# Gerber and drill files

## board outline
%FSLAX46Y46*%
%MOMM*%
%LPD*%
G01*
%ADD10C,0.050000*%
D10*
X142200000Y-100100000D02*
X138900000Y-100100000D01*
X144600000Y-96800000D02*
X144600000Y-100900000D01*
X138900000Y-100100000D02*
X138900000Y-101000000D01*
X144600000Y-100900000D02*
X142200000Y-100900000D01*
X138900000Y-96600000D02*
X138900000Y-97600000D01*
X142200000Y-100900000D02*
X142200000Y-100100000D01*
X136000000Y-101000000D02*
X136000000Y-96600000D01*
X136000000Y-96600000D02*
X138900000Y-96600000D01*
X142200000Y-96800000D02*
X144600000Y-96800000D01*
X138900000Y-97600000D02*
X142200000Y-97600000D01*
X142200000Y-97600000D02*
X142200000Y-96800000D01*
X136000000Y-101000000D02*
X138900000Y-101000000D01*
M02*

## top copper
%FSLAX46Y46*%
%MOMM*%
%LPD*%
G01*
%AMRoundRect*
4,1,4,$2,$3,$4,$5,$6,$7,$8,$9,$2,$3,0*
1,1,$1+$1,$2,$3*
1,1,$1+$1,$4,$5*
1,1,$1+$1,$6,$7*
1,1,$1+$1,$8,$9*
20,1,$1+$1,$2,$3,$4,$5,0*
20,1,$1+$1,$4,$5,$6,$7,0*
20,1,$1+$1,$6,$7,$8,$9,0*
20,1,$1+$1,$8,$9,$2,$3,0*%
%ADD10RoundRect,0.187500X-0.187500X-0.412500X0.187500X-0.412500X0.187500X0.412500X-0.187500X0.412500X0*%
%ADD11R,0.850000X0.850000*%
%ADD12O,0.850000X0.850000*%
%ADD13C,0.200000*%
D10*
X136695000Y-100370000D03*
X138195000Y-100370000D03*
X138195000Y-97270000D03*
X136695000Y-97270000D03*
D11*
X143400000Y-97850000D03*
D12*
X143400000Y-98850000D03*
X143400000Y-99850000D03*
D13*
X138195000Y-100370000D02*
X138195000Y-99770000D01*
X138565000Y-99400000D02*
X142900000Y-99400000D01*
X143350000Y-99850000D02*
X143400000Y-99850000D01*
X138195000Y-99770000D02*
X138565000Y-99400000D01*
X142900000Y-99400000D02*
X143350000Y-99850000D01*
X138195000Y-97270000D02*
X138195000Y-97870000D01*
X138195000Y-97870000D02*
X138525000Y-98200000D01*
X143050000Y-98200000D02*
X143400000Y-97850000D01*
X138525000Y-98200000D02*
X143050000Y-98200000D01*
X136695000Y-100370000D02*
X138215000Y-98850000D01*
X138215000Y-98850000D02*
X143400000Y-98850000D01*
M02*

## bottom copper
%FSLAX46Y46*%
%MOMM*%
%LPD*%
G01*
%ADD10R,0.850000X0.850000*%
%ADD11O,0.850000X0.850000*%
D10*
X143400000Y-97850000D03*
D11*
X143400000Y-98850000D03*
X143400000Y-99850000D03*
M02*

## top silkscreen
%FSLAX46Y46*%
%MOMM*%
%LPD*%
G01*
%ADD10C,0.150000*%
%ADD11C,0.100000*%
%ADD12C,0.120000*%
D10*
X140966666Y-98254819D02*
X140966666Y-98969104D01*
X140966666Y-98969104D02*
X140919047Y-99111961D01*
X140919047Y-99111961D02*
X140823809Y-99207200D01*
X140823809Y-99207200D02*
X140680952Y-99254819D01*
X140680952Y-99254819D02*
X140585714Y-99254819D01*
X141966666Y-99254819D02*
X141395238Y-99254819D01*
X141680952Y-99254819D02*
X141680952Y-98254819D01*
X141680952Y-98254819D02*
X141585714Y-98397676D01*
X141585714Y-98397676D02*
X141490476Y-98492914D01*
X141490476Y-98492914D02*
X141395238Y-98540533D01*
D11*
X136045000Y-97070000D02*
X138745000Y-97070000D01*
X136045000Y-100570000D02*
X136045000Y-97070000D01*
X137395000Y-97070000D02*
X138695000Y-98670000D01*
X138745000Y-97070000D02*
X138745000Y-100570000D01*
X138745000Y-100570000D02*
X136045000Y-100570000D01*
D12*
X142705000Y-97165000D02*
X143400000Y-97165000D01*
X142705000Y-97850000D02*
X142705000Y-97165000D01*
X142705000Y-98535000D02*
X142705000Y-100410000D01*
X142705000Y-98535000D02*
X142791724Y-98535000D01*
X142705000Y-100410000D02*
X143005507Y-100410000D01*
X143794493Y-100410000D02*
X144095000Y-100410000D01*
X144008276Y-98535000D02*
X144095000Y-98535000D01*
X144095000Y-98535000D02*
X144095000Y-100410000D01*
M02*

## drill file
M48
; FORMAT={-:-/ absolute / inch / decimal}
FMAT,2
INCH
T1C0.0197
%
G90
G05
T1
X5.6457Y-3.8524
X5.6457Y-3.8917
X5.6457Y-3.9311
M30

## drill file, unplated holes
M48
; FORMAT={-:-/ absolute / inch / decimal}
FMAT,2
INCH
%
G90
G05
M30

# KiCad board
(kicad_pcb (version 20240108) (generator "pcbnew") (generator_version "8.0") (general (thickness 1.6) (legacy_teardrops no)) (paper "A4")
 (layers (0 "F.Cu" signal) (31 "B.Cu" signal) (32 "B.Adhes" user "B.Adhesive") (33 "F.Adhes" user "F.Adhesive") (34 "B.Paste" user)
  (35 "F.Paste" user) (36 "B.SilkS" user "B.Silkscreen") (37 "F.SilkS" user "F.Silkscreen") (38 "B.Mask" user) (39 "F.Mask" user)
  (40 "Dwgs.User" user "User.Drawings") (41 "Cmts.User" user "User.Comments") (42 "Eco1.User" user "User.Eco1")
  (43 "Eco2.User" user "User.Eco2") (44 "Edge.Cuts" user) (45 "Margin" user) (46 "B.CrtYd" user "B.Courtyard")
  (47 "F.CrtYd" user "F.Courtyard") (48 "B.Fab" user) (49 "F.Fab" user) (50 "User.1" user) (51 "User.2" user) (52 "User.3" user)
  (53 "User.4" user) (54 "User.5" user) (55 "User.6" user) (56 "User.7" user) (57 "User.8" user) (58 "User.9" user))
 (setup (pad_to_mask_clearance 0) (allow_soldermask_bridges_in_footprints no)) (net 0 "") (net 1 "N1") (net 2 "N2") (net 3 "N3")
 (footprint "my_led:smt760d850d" (layer "F.Cu") (at 136.695 97.27)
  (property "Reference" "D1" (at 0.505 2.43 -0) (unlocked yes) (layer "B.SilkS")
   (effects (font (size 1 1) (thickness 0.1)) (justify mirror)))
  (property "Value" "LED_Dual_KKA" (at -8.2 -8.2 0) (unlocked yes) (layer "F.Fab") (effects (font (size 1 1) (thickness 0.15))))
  (fp_line (start -0.65 -0.2) (end 2.05 -0.2) (stroke (width 0.1) (type default)) (layer "F.SilkS"))
  (fp_line (start -0.65 3.3) (end -0.65 -0.2) (stroke (width 0.1) (type default)) (layer "F.SilkS"))
  (fp_line (start 0.7 -0.2) (end 2 1.4) (stroke (width 0.1) (type default)) (layer "F.SilkS"))
  (fp_line (start 2.05 -0.2) (end 2.05 3.3) (stroke (width 0.1) (type default)) (layer "F.SilkS"))
  (fp_line (start 2.05 3.3) (end -0.65 3.3) (stroke (width 0.1) (type default)) (layer "F.SilkS"))
  (pad "1" smd roundrect (at 0 3.1) (size 0.75 1.2) (layers "F.Cu" "F.Paste" "F.Mask") (roundrect_rratio 0.25) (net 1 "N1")
   (thermal_bridge_angle 45))
  (pad "2" smd roundrect (at 1.5 3.1) (size 0.75 1.2) (layers "F.Cu" "F.Paste" "F.Mask") (roundrect_rratio 0.25) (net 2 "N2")
   (thermal_bridge_angle 45))
  (pad "3" smd roundrect (at 1.5 0) (size 0.75 1.2) (layers "F.Cu" "F.Paste" "F.Mask") (roundrect_rratio 0.25) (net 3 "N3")
   (thermal_bridge_angle 45))
  (pad "4" smd roundrect (at 0 0) (size 0.75 1.2) (layers "F.Cu" "F.Paste" "F.Mask") (roundrect_rratio 0.25) (thermal_bridge_angle 45)))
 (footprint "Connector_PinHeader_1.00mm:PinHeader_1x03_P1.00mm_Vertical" (layer "F.Cu") (at 143.4 97.85)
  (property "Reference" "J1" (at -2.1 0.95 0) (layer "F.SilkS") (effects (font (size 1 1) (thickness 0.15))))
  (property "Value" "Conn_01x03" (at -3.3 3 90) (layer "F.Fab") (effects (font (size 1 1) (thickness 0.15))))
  (fp_line (start -0.695 -0.685) (end 0 -0.685) (stroke (width 0.12) (type solid)) (layer "F.SilkS"))
  (fp_line (start -0.695 0) (end -0.695 -0.685) (stroke (width 0.12) (type solid)) (layer "F.SilkS"))
  (fp_line (start -0.695 0.685) (end -0.695 2.56) (stroke (width 0.12) (type solid)) (layer "F.SilkS"))
  (fp_line (start -0.695 0.685) (end -0.608276 0.685) (stroke (width 0.12) (type solid)) (layer "F.SilkS"))
  (fp_line (start -0.695 2.56) (end -0.394493 2.56) (stroke (width 0.12) (type solid)) (layer "F.SilkS"))
  (fp_line (start 0.394493 2.56) (end 0.695 2.56) (stroke (width 0.12) (type solid)) (layer "F.SilkS"))
  (fp_line (start 0.608276 0.685) (end 0.695 0.685) (stroke (width 0.12) (type solid)) (layer "F.SilkS"))
  (fp_line (start 0.695 0.685) (end 0.695 2.56) (stroke (width 0.12) (type solid)) (layer "F.SilkS"))
  (pad "1" thru_hole rect (at 0 0) (size 0.85 0.85) (drill 0.5) (layers "*.Cu" "*.Mask") (remove_unused_layers no) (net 3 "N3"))
  (pad "2" thru_hole oval (at 0 1) (size 0.85 0.85) (drill 0.5) (layers "*.Cu" "*.Mask") (remove_unused_layers no) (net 1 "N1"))
  (pad "3" thru_hole oval (at 0 2) (size 0.85 0.85) (drill 0.5) (layers "*.Cu" "*.Mask") (remove_unused_layers no) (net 2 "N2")))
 (gr_line (start 142.2 100.1) (end 138.9 100.1) (stroke (width 0.05) (type default)) (layer "Edge.Cuts"))
 (gr_line (start 144.6 96.8) (end 144.6 100.9) (stroke (width 0.05) (type default)) (layer "Edge.Cuts"))
 (gr_line (start 138.9 100.1) (end 138.9 101) (stroke (width 0.05) (type default)) (layer "Edge.Cuts"))
 (gr_line (start 144.6 100.9) (end 142.2 100.9) (stroke (width 0.05) (type default)) (layer "Edge.Cuts"))
 (gr_line (start 138.9 96.6) (end 138.9 97.6) (stroke (width 0.05) (type default)) (layer "Edge.Cuts"))
 (gr_line (start 142.2 100.9) (end 142.2 100.1) (stroke (width 0.05) (type default)) (layer "Edge.Cuts"))
 (gr_line (start 136 101) (end 136 96.6) (stroke (width 0.05) (type default)) (layer "Edge.Cuts"))
 (gr_line (start 136 96.6) (end 138.9 96.6) (stroke (width 0.05) (type default)) (layer "Edge.Cuts"))
 (gr_line (start 142.2 96.8) (end 144.6 96.8) (stroke (width 0.05) (type default)) (layer "Edge.Cuts"))
 (gr_line (start 138.9 97.6) (end 142.2 97.6) (stroke (width 0.05) (type default)) (layer "Edge.Cuts"))
 (gr_line (start 142.2 97.6) (end 142.2 96.8) (stroke (width 0.05) (type default)) (layer "Edge.Cuts"))
 (gr_line (start 136 101) (end 138.9 101) (stroke (width 0.05) (type default)) (layer "Edge.Cuts"))
 (segment (start 138.195 100.37) (end 138.195 99.77) (width 0.2) (layer "F.Cu") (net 2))
 (segment (start 138.565 99.4) (end 142.9 99.4) (width 0.2) (layer "F.Cu") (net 2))
 (segment (start 143.35 99.85) (end 143.4 99.85) (width 0.2) (layer "F.Cu") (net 2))
 (segment (start 138.195 99.77) (end 138.565 99.4) (width 0.2) (layer "F.Cu") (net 2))
 (segment (start 142.9 99.4) (end 143.35 99.85) (width 0.2) (layer "F.Cu") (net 2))
 (segment (start 138.195 97.27) (end 138.195 97.87) (width 0.2) (layer "F.Cu") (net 3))
 (segment (start 138.195 97.87) (end 138.525 98.2) (width 0.2) (layer "F.Cu") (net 3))
 (segment (start 143.05 98.2) (end 143.4 97.85) (width 0.2) (layer "F.Cu") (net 3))
 (segment (start 138.525 98.2) (end 143.05 98.2) (width 0.2) (layer "F.Cu") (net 3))
 (segment (start 136.695 100.37) (end 138.215 98.85) (width 0.2) (layer "F.Cu") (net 1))
 (segment (start 138.215 98.85) (end 143.4 98.85) (width 0.2) (layer "F.Cu") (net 1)))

